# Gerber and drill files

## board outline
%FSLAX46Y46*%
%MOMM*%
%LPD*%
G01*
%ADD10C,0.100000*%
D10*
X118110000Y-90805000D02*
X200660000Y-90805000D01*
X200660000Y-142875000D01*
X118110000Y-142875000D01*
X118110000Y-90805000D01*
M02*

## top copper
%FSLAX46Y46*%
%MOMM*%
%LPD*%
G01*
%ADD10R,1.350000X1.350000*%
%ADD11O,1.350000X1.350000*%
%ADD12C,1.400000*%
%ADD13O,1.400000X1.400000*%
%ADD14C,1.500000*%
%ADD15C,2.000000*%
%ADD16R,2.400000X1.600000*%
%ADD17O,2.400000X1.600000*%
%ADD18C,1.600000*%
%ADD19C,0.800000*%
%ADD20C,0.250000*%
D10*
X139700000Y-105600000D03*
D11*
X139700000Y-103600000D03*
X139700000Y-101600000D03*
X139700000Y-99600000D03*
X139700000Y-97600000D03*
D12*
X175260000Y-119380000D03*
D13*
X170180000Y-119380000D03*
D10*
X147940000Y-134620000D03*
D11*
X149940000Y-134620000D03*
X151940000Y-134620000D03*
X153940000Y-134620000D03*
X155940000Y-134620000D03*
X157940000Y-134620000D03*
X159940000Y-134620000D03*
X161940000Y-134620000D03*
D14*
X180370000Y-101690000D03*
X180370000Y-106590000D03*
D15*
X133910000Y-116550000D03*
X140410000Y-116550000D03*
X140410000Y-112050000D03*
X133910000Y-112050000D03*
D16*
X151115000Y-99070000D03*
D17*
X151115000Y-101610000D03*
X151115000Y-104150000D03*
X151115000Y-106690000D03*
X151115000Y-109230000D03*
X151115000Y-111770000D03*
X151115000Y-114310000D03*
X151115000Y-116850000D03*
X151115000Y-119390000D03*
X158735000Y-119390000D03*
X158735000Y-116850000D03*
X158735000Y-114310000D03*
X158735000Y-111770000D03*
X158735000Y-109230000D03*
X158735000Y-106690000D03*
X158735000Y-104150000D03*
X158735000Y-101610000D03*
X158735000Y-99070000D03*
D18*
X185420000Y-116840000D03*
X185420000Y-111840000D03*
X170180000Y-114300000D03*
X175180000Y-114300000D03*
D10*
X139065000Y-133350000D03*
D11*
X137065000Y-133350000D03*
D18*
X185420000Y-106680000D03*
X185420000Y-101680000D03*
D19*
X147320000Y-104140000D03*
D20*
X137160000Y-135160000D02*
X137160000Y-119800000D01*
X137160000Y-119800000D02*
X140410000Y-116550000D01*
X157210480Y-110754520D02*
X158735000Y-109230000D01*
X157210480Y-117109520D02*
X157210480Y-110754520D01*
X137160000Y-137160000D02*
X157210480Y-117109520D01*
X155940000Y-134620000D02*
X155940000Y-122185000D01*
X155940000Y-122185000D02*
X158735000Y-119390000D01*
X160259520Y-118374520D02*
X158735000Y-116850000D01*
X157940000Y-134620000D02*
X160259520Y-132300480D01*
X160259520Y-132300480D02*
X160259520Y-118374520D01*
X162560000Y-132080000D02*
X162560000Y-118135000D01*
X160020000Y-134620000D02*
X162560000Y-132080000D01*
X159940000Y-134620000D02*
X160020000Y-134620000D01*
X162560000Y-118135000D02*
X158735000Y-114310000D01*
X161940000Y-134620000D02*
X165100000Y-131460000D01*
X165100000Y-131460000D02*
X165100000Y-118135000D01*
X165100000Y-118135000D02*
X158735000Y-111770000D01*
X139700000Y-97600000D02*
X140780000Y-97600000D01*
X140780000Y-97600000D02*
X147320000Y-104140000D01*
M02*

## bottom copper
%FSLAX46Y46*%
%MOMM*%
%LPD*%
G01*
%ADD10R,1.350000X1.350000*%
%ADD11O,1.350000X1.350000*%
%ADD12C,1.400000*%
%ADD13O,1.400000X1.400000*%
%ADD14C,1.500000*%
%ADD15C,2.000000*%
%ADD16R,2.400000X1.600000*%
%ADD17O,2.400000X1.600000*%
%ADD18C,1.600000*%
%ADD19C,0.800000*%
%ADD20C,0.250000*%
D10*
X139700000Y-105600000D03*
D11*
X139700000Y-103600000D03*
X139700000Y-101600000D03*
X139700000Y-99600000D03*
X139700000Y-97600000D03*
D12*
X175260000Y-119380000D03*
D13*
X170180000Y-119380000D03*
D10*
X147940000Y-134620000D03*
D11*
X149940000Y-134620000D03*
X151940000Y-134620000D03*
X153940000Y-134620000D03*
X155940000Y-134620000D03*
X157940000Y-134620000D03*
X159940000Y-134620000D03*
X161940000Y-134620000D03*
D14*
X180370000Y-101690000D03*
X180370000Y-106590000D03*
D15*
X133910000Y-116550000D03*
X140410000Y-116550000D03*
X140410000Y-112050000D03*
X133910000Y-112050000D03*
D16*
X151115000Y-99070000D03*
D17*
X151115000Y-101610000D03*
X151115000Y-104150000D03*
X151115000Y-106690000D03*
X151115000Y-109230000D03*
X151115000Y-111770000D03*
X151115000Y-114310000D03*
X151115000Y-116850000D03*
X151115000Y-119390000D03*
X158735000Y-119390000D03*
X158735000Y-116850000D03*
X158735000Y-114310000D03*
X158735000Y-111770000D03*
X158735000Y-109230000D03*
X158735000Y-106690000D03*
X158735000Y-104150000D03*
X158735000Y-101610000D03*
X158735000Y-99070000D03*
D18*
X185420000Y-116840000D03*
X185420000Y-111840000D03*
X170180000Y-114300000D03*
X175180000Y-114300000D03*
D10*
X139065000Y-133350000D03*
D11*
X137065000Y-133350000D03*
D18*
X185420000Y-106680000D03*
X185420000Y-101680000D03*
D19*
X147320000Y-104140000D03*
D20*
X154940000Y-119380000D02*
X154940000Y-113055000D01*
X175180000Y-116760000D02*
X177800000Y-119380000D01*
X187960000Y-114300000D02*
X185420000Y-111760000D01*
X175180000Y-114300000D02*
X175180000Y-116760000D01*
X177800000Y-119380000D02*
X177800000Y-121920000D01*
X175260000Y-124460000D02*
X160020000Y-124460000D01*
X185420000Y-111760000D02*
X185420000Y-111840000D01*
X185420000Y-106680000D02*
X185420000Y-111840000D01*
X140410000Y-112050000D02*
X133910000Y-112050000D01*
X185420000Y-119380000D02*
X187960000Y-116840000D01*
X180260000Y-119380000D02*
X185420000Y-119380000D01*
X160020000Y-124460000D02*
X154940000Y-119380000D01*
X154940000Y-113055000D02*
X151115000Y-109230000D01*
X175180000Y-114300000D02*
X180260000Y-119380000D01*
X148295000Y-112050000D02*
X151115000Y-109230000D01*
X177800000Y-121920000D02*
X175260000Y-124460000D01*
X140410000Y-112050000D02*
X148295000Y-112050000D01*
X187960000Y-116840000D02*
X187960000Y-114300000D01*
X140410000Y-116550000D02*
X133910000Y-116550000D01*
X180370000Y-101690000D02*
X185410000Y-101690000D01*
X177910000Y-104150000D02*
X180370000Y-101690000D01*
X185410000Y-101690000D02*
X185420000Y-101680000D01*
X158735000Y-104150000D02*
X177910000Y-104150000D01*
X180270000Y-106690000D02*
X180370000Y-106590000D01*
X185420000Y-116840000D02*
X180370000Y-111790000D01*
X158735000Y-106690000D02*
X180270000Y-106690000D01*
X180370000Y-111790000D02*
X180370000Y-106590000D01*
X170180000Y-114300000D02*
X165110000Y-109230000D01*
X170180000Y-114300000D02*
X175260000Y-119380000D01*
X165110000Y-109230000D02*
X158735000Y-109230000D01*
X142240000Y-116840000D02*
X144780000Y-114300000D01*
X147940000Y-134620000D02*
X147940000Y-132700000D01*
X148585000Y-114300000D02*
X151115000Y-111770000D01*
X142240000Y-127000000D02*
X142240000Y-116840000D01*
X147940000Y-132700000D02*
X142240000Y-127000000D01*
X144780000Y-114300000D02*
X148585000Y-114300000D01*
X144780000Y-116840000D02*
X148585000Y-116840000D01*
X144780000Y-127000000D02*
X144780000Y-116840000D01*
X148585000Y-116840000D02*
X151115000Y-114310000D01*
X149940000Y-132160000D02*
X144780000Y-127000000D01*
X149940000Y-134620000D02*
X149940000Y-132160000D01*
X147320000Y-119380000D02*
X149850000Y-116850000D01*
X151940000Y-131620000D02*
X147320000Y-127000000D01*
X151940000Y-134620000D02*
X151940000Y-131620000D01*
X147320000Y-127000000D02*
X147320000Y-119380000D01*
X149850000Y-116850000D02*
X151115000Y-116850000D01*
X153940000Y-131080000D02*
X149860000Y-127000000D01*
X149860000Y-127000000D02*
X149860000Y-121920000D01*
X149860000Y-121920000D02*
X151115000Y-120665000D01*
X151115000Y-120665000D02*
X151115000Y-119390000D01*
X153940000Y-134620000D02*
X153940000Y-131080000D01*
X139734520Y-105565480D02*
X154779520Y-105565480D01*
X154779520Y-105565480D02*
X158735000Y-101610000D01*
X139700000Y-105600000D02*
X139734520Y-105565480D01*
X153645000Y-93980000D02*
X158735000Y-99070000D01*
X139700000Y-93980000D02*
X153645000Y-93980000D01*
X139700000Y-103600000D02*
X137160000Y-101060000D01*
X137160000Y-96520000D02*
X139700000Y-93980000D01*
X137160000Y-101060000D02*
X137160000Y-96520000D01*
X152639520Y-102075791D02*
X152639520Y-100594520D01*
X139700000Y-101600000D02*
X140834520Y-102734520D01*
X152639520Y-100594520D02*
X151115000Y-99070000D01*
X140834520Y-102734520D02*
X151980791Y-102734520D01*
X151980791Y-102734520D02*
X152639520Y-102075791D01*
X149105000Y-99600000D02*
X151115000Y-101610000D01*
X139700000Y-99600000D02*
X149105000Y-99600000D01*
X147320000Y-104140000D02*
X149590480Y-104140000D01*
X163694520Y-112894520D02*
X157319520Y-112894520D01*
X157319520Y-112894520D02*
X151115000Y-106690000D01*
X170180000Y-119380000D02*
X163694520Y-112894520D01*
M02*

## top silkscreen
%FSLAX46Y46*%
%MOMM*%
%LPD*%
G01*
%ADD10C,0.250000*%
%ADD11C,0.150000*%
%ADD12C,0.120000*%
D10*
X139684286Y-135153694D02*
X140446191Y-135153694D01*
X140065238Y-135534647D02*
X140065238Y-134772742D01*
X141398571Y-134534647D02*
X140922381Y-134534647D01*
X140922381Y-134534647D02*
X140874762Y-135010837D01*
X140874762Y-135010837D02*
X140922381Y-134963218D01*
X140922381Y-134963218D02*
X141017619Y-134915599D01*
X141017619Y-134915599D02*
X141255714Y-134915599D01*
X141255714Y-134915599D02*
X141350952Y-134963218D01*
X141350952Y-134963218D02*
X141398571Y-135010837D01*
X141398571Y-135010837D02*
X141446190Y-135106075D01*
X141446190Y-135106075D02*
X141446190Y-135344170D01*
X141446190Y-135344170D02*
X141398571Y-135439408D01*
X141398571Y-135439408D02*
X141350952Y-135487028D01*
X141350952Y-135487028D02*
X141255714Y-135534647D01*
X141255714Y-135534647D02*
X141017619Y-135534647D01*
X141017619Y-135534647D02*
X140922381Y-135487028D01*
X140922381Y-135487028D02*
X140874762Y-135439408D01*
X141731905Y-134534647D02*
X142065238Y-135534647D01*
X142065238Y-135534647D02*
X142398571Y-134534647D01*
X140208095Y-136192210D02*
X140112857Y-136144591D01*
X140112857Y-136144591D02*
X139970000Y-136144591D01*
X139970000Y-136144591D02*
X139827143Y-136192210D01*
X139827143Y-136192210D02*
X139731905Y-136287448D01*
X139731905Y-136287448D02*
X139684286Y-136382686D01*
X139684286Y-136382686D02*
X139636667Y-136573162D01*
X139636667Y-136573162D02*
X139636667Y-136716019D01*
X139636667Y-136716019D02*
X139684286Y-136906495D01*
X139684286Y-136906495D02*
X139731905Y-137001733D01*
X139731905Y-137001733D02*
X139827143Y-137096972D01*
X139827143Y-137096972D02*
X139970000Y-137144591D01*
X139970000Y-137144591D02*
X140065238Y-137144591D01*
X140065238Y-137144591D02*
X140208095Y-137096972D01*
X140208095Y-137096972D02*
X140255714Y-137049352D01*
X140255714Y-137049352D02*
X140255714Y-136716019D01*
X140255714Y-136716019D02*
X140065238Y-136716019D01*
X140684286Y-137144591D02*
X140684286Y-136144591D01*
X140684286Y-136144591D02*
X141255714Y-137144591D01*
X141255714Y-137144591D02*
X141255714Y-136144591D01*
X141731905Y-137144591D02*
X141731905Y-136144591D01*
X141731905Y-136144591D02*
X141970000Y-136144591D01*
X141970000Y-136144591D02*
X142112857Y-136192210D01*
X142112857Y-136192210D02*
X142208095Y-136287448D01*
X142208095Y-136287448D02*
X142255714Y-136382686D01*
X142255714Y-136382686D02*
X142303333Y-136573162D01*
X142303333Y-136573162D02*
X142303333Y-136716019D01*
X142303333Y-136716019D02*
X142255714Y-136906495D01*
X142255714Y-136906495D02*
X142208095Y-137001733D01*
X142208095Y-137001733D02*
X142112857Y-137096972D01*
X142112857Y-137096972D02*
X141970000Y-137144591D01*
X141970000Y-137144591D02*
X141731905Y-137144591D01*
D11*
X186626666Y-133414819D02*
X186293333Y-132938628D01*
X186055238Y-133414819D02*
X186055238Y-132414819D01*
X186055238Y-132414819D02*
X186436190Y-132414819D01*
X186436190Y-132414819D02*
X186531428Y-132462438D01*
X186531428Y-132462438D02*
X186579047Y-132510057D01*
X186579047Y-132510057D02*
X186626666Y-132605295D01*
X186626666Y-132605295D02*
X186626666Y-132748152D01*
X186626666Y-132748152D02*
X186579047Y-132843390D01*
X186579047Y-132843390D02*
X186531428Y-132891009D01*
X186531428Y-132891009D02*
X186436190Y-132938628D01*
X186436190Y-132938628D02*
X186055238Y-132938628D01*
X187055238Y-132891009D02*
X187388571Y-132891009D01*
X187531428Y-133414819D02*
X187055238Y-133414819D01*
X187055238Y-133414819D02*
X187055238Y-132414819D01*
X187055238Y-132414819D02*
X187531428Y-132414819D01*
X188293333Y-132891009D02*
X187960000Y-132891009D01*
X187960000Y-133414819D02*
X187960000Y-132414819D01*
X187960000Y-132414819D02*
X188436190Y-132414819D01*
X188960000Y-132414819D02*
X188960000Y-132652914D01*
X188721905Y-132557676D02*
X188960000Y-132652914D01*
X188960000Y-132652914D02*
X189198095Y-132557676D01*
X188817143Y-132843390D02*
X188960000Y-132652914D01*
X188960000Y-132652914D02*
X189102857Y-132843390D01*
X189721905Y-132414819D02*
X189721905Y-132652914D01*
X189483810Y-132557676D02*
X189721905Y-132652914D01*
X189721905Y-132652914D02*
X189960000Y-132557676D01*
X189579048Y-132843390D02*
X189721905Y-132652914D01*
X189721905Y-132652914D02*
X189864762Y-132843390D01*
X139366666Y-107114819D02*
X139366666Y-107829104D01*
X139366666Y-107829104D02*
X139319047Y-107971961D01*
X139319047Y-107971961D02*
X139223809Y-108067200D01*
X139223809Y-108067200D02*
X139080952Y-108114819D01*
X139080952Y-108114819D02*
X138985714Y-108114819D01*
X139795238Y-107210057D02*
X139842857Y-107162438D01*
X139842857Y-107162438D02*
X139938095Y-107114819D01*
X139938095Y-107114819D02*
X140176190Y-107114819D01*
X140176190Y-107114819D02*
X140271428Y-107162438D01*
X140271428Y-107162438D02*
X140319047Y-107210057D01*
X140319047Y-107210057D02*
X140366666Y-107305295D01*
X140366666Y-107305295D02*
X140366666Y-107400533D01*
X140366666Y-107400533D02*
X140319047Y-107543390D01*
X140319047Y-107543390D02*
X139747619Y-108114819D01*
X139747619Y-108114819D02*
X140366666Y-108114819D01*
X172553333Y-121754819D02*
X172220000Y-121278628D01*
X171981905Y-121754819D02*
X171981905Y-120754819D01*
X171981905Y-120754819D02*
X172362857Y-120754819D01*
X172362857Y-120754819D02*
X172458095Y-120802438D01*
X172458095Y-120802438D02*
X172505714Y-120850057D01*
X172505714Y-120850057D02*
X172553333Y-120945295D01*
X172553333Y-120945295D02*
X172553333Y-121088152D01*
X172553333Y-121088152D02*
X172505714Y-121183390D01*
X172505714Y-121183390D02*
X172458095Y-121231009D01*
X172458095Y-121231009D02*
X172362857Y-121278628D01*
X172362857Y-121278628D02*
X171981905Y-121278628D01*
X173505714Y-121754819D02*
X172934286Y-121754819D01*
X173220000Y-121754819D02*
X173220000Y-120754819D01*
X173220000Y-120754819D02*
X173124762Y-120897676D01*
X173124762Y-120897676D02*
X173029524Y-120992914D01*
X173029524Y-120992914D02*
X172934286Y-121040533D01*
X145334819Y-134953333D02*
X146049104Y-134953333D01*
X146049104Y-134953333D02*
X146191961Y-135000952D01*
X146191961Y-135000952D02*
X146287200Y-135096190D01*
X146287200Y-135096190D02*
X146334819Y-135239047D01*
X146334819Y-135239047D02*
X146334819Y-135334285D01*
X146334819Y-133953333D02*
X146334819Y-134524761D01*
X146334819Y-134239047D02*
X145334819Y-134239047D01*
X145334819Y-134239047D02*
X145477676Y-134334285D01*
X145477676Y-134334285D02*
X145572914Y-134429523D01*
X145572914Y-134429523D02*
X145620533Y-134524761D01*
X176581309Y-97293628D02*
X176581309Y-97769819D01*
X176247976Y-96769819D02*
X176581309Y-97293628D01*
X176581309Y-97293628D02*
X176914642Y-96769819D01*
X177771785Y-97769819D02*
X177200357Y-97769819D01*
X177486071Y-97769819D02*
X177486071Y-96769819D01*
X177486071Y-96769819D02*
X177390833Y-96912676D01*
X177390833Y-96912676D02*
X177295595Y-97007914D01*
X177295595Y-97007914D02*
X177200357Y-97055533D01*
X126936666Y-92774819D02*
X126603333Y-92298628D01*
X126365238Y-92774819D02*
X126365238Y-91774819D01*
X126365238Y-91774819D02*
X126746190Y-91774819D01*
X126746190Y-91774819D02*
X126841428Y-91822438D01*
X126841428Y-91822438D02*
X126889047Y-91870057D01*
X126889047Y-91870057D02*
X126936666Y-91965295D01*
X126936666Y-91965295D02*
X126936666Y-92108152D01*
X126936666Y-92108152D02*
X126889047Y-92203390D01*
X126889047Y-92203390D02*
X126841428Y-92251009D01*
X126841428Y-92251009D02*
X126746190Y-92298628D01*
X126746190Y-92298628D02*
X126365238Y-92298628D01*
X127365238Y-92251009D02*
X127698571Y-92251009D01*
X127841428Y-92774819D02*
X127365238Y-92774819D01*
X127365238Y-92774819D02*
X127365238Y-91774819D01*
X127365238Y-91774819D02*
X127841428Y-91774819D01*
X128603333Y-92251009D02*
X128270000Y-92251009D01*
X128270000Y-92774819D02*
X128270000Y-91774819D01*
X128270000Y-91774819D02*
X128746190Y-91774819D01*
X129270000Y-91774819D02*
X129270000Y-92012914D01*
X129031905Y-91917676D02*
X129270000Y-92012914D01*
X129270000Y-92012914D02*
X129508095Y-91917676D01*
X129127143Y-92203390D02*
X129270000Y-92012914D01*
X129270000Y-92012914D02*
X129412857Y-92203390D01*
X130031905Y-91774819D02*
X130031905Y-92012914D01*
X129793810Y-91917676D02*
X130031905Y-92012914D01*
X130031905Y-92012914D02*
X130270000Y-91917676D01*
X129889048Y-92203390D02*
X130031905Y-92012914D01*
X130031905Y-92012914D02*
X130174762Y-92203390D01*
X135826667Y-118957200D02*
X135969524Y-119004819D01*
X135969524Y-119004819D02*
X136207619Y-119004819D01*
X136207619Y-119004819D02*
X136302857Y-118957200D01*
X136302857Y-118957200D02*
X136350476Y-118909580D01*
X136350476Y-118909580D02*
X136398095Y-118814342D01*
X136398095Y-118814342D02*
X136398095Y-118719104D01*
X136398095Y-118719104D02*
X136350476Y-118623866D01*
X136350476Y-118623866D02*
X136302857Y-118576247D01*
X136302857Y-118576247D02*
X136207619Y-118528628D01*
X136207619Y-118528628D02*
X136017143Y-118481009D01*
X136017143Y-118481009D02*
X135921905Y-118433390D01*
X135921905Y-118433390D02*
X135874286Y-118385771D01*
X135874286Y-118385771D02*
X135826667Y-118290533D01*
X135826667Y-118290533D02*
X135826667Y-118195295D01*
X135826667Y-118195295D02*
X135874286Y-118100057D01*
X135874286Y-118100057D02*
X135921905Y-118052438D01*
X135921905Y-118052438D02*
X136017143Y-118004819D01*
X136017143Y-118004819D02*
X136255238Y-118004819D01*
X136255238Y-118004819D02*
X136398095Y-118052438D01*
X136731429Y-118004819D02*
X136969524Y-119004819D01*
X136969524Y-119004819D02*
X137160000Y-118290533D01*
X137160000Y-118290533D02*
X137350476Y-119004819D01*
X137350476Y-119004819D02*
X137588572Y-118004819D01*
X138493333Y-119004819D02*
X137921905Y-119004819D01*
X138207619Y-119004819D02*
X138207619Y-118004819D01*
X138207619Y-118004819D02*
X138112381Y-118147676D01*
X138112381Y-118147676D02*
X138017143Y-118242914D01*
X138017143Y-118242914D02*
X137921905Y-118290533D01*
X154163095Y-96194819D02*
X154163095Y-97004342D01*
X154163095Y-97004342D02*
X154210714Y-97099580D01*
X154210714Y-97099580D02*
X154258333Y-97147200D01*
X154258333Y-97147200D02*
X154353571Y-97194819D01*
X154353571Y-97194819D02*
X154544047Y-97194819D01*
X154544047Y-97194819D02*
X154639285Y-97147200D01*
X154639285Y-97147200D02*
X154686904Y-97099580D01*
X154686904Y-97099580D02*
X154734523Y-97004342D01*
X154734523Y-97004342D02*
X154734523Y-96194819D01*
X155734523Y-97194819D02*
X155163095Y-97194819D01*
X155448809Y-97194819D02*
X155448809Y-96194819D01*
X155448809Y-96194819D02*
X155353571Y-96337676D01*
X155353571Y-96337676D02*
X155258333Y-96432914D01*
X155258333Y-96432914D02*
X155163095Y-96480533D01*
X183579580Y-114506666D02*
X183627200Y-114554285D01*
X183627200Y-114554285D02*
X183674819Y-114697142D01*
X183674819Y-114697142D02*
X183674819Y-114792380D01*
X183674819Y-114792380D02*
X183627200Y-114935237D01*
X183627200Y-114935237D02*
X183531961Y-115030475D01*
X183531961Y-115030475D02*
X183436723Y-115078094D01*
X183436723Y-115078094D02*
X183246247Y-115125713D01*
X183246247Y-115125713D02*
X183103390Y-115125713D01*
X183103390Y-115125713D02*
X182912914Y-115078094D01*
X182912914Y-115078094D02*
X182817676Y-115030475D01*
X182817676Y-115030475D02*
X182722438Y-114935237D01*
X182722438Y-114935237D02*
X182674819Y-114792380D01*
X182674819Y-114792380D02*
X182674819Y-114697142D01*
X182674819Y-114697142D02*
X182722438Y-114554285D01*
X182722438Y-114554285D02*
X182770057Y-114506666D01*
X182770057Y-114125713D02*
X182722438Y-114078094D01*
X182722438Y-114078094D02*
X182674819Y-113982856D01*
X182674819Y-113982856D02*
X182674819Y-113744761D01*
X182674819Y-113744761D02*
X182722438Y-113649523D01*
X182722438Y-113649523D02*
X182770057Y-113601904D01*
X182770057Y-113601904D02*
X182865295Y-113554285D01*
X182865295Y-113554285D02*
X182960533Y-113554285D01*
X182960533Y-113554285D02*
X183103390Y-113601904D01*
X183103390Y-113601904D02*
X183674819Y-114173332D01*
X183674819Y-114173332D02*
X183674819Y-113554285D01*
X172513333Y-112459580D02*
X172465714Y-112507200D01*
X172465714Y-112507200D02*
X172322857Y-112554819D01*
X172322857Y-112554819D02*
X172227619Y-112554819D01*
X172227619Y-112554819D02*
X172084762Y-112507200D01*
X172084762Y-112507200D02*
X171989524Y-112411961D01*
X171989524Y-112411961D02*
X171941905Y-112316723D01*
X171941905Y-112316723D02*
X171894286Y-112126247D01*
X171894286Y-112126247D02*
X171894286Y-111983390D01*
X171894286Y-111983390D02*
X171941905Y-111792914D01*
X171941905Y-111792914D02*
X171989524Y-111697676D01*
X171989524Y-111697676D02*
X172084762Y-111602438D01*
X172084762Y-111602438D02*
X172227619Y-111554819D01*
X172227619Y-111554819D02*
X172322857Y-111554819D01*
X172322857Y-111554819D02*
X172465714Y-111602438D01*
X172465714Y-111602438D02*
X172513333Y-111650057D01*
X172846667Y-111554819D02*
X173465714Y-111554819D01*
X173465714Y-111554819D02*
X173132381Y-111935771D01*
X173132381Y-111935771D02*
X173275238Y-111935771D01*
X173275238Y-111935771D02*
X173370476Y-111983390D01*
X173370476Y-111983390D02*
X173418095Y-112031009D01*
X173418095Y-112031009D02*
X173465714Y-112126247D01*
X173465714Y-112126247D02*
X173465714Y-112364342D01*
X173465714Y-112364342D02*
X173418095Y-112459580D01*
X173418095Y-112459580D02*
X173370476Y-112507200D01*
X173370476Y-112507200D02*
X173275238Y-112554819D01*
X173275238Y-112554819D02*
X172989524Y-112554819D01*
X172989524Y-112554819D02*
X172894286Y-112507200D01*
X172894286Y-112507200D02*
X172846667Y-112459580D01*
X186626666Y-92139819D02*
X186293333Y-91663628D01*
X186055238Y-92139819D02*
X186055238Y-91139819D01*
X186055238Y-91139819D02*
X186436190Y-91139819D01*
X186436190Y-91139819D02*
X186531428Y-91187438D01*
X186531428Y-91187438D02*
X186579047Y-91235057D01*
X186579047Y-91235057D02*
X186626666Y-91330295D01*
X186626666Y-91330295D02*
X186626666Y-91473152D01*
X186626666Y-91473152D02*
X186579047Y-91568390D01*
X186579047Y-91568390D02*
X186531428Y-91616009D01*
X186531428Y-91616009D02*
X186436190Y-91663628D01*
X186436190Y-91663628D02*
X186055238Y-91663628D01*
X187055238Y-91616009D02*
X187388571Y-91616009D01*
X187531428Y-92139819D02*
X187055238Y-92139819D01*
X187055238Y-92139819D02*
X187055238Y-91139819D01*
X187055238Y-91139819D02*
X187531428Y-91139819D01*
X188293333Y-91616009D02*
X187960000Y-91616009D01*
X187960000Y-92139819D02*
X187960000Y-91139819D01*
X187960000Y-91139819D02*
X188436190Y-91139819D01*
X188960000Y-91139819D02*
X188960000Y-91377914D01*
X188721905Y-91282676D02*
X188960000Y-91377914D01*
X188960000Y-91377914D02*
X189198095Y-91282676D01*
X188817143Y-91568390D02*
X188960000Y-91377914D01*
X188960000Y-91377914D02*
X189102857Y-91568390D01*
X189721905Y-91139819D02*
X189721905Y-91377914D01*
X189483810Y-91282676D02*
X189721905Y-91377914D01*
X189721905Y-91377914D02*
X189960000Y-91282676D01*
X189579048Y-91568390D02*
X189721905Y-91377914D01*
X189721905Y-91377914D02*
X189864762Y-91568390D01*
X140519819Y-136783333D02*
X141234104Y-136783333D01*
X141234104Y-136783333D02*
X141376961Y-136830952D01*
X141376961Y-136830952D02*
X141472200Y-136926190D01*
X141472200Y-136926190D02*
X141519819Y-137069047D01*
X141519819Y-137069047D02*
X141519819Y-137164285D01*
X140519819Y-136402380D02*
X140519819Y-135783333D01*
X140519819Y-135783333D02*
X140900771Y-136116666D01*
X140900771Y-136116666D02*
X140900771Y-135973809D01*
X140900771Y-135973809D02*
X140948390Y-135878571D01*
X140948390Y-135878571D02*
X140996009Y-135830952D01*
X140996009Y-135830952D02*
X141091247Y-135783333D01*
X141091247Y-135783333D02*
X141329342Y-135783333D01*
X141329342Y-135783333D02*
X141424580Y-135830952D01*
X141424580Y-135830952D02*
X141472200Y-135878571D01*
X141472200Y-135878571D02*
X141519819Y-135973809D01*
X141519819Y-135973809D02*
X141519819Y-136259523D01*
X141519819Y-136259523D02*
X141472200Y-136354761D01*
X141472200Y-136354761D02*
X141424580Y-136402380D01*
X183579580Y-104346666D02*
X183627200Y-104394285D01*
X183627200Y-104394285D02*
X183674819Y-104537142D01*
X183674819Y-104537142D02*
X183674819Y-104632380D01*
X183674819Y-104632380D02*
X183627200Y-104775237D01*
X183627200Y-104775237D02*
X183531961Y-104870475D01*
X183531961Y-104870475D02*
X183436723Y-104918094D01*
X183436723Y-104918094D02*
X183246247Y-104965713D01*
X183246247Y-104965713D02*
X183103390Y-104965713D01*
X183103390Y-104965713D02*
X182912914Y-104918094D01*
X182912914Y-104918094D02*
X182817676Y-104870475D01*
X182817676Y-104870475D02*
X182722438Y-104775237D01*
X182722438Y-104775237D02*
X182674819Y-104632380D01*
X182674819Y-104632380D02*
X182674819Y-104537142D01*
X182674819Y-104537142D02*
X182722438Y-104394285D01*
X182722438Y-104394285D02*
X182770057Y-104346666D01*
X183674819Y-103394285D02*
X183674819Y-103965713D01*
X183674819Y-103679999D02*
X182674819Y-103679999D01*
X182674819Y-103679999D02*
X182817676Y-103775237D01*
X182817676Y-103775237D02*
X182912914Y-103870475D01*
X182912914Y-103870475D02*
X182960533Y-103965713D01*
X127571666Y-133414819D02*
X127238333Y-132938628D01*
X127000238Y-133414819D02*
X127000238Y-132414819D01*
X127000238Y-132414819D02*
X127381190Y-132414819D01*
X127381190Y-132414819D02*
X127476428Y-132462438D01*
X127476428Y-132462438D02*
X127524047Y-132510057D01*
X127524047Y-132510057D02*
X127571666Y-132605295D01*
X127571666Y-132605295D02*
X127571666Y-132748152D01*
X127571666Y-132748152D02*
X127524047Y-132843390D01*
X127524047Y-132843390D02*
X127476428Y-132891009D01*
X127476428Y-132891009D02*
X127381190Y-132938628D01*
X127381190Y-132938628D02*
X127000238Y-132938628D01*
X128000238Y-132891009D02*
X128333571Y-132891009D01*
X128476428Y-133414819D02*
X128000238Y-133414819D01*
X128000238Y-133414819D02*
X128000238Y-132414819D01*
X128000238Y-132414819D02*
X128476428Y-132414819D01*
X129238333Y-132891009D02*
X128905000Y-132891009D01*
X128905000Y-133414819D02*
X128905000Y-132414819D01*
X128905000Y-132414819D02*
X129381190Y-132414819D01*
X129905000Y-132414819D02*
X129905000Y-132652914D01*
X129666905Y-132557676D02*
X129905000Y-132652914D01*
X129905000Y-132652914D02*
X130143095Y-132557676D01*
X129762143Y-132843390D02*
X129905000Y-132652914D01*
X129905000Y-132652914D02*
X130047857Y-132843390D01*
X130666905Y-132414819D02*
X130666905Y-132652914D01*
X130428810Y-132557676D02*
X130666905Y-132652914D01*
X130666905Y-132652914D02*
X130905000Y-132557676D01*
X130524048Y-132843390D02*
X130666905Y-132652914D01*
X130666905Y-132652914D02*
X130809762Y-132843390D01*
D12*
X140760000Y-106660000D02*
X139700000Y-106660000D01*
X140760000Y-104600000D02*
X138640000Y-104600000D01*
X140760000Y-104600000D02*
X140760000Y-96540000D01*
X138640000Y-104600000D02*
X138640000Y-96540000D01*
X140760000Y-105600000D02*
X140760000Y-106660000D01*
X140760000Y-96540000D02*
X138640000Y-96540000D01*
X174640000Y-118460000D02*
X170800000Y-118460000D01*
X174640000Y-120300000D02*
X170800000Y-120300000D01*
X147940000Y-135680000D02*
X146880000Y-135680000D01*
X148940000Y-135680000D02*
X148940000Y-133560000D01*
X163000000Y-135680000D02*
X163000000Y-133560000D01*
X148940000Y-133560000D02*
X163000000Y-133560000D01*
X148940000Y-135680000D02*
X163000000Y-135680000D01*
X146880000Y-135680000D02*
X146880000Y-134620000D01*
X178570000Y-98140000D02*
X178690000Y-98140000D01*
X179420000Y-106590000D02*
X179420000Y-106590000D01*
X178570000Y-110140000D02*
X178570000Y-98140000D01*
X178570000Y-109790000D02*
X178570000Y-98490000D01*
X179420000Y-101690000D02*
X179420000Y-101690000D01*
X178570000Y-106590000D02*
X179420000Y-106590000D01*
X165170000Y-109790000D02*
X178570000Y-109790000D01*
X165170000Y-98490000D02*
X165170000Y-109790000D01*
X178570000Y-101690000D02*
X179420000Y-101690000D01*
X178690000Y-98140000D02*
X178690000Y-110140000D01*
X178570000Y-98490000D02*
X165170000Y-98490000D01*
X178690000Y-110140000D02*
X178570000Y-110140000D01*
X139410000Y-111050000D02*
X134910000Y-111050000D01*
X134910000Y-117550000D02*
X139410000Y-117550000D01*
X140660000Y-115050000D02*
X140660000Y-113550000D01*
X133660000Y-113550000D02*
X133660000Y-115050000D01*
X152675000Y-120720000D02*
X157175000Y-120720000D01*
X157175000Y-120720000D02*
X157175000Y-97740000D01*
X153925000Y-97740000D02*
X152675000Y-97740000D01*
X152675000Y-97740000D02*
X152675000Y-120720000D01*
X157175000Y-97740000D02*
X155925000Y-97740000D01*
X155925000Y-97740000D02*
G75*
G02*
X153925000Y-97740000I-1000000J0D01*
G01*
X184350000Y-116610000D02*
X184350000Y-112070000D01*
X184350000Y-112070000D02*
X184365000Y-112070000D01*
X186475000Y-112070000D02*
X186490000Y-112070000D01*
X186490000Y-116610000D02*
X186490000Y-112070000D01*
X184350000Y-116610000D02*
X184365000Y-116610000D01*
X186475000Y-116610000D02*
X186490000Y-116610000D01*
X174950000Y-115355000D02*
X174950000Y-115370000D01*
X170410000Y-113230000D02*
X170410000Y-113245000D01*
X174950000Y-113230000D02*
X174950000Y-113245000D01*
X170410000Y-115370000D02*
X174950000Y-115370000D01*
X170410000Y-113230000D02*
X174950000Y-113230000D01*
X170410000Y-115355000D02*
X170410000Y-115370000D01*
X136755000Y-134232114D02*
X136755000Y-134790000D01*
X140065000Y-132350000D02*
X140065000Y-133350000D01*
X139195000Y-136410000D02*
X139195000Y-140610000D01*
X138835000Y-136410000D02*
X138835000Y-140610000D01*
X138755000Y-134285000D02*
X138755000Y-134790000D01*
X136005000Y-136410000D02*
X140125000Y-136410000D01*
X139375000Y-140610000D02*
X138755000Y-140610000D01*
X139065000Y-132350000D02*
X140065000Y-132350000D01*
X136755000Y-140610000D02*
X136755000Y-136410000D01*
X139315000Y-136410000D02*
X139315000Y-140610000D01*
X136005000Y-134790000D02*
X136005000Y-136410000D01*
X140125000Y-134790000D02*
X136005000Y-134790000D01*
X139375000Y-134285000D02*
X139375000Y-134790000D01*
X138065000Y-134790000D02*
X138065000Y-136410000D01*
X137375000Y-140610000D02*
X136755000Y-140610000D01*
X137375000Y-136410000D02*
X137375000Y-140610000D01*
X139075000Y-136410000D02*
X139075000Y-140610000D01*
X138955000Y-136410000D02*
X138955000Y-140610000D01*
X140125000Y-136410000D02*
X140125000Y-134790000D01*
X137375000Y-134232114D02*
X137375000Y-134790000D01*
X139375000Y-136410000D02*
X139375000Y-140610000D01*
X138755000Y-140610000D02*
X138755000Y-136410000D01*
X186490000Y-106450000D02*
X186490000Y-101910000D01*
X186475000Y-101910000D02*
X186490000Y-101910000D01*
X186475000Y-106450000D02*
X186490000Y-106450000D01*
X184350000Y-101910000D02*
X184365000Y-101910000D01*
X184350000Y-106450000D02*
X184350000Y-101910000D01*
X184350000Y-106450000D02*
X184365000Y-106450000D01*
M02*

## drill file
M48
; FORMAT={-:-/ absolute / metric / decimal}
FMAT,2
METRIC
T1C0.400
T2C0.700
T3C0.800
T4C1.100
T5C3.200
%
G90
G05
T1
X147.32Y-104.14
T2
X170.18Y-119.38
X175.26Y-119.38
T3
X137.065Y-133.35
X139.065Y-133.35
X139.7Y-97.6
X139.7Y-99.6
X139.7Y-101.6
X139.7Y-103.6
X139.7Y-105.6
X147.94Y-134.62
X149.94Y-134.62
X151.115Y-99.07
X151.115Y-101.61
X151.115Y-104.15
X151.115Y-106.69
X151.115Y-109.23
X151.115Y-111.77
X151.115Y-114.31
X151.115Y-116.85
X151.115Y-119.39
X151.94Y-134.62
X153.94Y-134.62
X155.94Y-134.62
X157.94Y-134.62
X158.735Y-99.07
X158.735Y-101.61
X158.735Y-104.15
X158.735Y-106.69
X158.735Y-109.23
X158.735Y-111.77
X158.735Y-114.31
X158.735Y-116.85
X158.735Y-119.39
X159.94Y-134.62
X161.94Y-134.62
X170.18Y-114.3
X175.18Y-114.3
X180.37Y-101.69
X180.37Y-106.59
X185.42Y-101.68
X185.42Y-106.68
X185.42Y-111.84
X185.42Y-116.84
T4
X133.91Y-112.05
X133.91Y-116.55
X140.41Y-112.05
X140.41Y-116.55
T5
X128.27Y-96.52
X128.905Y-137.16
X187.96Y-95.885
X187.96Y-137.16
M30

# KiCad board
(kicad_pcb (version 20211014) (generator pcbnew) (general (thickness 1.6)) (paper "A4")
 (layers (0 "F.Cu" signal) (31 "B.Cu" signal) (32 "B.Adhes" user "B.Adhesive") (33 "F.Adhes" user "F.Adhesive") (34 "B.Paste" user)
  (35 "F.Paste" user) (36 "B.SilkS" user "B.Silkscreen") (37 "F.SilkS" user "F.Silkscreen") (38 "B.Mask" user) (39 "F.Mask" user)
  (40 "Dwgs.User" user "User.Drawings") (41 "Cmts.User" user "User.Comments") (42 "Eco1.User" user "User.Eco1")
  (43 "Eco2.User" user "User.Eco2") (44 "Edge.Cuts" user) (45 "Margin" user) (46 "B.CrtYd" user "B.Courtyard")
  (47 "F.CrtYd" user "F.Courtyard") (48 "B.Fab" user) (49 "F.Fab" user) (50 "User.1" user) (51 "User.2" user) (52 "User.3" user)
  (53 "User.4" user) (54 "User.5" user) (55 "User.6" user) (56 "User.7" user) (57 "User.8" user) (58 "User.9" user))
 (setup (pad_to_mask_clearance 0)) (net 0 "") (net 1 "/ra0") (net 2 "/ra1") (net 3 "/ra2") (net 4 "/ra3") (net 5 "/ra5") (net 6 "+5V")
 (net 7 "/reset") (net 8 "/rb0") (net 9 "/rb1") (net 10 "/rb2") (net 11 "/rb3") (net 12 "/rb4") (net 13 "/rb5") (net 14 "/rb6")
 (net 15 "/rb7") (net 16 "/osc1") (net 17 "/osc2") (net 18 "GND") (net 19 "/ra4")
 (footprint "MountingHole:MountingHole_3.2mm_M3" (layer "F.Cu") (at 187.96 137.16)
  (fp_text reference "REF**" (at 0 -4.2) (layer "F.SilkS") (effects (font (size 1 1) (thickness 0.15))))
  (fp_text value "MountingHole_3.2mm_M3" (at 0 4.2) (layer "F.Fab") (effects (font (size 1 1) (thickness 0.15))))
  (pad "" np_thru_hole circle (at 0 0) (size 3.2 3.2) (drill 3.2) (layers *.Cu *.Mask)))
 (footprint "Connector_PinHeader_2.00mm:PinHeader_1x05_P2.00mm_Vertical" (layer "F.Cu") (at 139.7 105.6 180)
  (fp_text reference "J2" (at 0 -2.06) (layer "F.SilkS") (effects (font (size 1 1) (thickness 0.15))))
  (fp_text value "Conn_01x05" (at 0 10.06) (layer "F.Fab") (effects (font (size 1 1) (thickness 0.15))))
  (fp_line (start -1.06 -1.06) (end 0 -1.06) (layer "F.SilkS") (width 0.12))
  (fp_line (start -1.06 1) (end 1.06 1) (layer "F.SilkS") (width 0.12))
  (fp_line (start -1.06 1) (end -1.06 9.06) (layer "F.SilkS") (width 0.12))
  (fp_line (start 1.06 1) (end 1.06 9.06) (layer "F.SilkS") (width 0.12))
  (fp_line (start -1.06 0) (end -1.06 -1.06) (layer "F.SilkS") (width 0.12))
  (fp_line (start -1.06 9.06) (end 1.06 9.06) (layer "F.SilkS") (width 0.12))
  (pad "1" thru_hole rect (at 0 0 180) (size 1.35 1.35) (drill 0.8) (layers *.Cu *.Mask) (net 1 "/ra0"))
  (pad "2" thru_hole oval (at 0 2 180) (size 1.35 1.35) (drill 0.8) (layers *.Cu *.Mask) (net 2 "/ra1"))
  (pad "3" thru_hole oval (at 0 4 180) (size 1.35 1.35) (drill 0.8) (layers *.Cu *.Mask) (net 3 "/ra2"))
  (pad "4" thru_hole oval (at 0 6 180) (size 1.35 1.35) (drill 0.8) (layers *.Cu *.Mask) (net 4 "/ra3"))
  (pad "5" thru_hole oval (at 0 8 180) (size 1.35 1.35) (drill 0.8) (layers *.Cu *.Mask) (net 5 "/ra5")))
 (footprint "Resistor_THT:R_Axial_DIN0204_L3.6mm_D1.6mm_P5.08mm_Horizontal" (layer "F.Cu") (at 175.26 119.38 180)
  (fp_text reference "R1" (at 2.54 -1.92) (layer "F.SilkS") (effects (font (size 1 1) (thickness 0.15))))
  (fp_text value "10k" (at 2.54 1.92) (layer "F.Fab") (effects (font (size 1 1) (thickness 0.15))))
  (fp_line (start 0.62 0.92) (end 4.46 0.92) (layer "F.SilkS") (width 0.12))
  (fp_line (start 0.62 -0.92) (end 4.46 -0.92) (layer "F.SilkS") (width 0.12))
  (pad "1" thru_hole circle (at 0 0 180) (size 1.4 1.4) (drill 0.7) (layers *.Cu *.Mask) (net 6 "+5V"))
  (pad "2" thru_hole oval (at 5.08 0 180) (size 1.4 1.4) (drill 0.7) (layers *.Cu *.Mask) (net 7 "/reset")))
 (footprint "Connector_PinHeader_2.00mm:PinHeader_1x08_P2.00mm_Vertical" (layer "F.Cu") (at 147.94 134.62 90)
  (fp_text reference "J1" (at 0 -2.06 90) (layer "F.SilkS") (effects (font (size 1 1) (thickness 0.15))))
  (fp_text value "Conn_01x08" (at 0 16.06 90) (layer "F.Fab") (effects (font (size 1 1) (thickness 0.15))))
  (fp_line (start -1.06 0) (end -1.06 -1.06) (layer "F.SilkS") (width 0.12))
  (fp_line (start -1.06 1) (end 1.06 1) (layer "F.SilkS") (width 0.12))
  (fp_line (start -1.06 15.06) (end 1.06 15.06) (layer "F.SilkS") (width 0.12))
  (fp_line (start 1.06 1) (end 1.06 15.06) (layer "F.SilkS") (width 0.12))
  (fp_line (start -1.06 1) (end -1.06 15.06) (layer "F.SilkS") (width 0.12))
  (fp_line (start -1.06 -1.06) (end 0 -1.06) (layer "F.SilkS") (width 0.12))
  (pad "1" thru_hole rect (at 0 0 90) (size 1.35 1.35) (drill 0.8) (layers *.Cu *.Mask) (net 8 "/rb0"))
  (pad "2" thru_hole oval (at 0 2 90) (size 1.35 1.35) (drill 0.8) (layers *.Cu *.Mask) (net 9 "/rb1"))
  (pad "3" thru_hole oval (at 0 4 90) (size 1.35 1.35) (drill 0.8) (layers *.Cu *.Mask) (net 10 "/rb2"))
  (pad "4" thru_hole oval (at 0 6 90) (size 1.35 1.35) (drill 0.8) (layers *.Cu *.Mask) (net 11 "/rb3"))
  (pad "5" thru_hole oval (at 0 8 90) (size 1.35 1.35) (drill 0.8) (layers *.Cu *.Mask) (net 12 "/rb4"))
  (pad "6" thru_hole oval (at 0 10 90) (size 1.35 1.35) (drill 0.8) (layers *.Cu *.Mask) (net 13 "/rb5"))
  (pad "7" thru_hole oval (at 0 12 90) (size 1.35 1.35) (drill 0.8) (layers *.Cu *.Mask) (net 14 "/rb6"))
  (pad "8" thru_hole oval (at 0 14 90) (size 1.35 1.35) (drill 0.8) (layers *.Cu *.Mask) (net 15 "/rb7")))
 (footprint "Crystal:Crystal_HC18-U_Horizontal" (layer "F.Cu") (at 180.37 101.69 -90)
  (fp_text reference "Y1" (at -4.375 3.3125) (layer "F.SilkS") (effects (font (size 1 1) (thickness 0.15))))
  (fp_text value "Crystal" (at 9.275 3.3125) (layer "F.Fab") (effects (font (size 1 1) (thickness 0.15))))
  (fp_line (start -3.55 1.8) (end -3.55 1.68) (layer "F.SilkS") (width 0.12))
  (fp_line (start 4.9 0.95) (end 4.9 0.95) (layer "F.SilkS") (width 0.12))
  (fp_line (start 8.45 1.8) (end -3.55 1.8) (layer "F.SilkS") (width 0.12))
  (fp_line (start 8.1 1.8) (end -3.2 1.8) (layer "F.SilkS") (width 0.12))
  (fp_line (start 0 0.95) (end 0 0.95) (layer "F.SilkS") (width 0.12))
  (fp_line (start 4.9 1.8) (end 4.9 0.95) (layer "F.SilkS") (width 0.12))
  (fp_line (start 8.1 15.2) (end 8.1 1.8) (layer "F.SilkS") (width 0.12))
  (fp_line (start -3.2 15.2) (end 8.1 15.2) (layer "F.SilkS") (width 0.12))
  (fp_line (start 0 1.8) (end 0 0.95) (layer "F.SilkS") (width 0.12))
  (fp_line (start -3.55 1.68) (end 8.45 1.68) (layer "F.SilkS") (width 0.12))
  (fp_line (start -3.2 1.8) (end -3.2 15.2) (layer "F.SilkS") (width 0.12))
  (fp_line (start 8.45 1.68) (end 8.45 1.8) (layer "F.SilkS") (width 0.12))
  (pad "1" thru_hole circle (at 0 0 270) (size 1.5 1.5) (drill 0.8) (layers *.Cu *.Mask) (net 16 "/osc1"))
  (pad "2" thru_hole circle (at 4.9 0 270) (size 1.5 1.5) (drill 0.8) (layers *.Cu *.Mask) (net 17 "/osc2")))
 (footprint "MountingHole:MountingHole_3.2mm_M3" (layer "F.Cu") (at 128.27 96.52)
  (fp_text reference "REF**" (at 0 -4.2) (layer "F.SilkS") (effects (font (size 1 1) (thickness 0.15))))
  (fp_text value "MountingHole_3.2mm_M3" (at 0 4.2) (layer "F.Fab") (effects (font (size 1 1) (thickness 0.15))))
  (pad "" np_thru_hole circle (at 0 0) (size 3.2 3.2) (drill 3.2) (layers *.Cu *.Mask)))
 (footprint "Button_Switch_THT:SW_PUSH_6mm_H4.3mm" (layer "F.Cu") (at 140.41 116.55 180)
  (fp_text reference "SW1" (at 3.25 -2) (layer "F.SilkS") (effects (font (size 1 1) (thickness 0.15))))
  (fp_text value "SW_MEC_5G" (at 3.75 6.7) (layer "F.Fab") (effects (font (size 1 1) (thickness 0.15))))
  (fp_line (start 1 5.5) (end 5.5 5.5) (layer "F.SilkS") (width 0.12))
  (fp_line (start 5.5 -1) (end 1 -1) (layer "F.SilkS") (width 0.12))
  (fp_line (start -0.25 1.5) (end -0.25 3) (layer "F.SilkS") (width 0.12))
  (fp_line (start 6.75 3) (end 6.75 1.5) (layer "F.SilkS") (width 0.12))
  (pad "1" thru_hole circle (at 6.5 0 270) (size 2 2) (drill 1.1) (layers *.Cu *.Mask) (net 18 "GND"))
  (pad "1" thru_hole circle (at 0 0 270) (size 2 2) (drill 1.1) (layers *.Cu *.Mask) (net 18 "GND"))
  (pad "2" thru_hole circle (at 0 4.5 270) (size 2 2) (drill 1.1) (layers *.Cu *.Mask) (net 18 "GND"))
  (pad "2" thru_hole circle (at 6.5 4.5 270) (size 2 2) (drill 1.1) (layers *.Cu *.Mask) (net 18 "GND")))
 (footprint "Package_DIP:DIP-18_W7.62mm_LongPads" (layer "F.Cu") (at 151.115 99.07)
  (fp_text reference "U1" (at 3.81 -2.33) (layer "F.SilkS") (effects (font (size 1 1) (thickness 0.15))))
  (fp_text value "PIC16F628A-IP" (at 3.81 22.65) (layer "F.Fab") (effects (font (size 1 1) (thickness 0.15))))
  (fp_line (start 1.56 21.65) (end 6.06 21.65) (layer "F.SilkS") (width 0.12))
  (fp_line (start 6.06 21.65) (end 6.06 -1.33) (layer "F.SilkS") (width 0.12))
  (fp_line (start 2.81 -1.33) (end 1.56 -1.33) (layer "F.SilkS") (width 0.12))
  (fp_line (start 1.56 -1.33) (end 1.56 21.65) (layer "F.SilkS") (width 0.12))
  (fp_line (start 6.06 -1.33) (end 4.81 -1.33) (layer "F.SilkS") (width 0.12))
  (fp_arc (start 4.81 -1.33) (mid 3.81 -0.33) (end 2.81 -1.33) (layer "F.SilkS") (width 0.12))
  (pad "1" thru_hole rect (at 0 0) (size 2.4 1.6) (drill 0.8) (layers *.Cu *.Mask) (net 3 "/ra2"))
  (pad "2" thru_hole oval (at 0 2.54) (size 2.4 1.6) (drill 0.8) (layers *.Cu *.Mask) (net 4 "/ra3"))
  (pad "3" thru_hole oval (at 0 5.08) (size 2.4 1.6) (drill 0.8) (layers *.Cu *.Mask) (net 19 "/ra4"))
  (pad "4" thru_hole oval (at 0 7.62) (size 2.4 1.6) (drill 0.8) (layers *.Cu *.Mask) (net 7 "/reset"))
  (pad "5" thru_hole oval (at 0 10.16) (size 2.4 1.6) (drill 0.8) (layers *.Cu *.Mask) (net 18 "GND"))
  (pad "6" thru_hole oval (at 0 12.7) (size 2.4 1.6) (drill 0.8) (layers *.Cu *.Mask) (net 8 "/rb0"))
  (pad "7" thru_hole oval (at 0 15.24) (size 2.4 1.6) (drill 0.8) (layers *.Cu *.Mask) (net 9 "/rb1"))
  (pad "8" thru_hole oval (at 0 17.78) (size 2.4 1.6) (drill 0.8) (layers *.Cu *.Mask) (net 10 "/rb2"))
  (pad "9" thru_hole oval (at 0 20.32) (size 2.4 1.6) (drill 0.8) (layers *.Cu *.Mask) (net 11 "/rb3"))
  (pad "10" thru_hole oval (at 7.62 20.32) (size 2.4 1.6) (drill 0.8) (layers *.Cu *.Mask) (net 12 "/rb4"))
  (pad "11" thru_hole oval (at 7.62 17.78) (size 2.4 1.6) (drill 0.8) (layers *.Cu *.Mask) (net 13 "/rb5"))
  (pad "12" thru_hole oval (at 7.62 15.24) (size 2.4 1.6) (drill 0.8) (layers *.Cu *.Mask) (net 14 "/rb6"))
  (pad "13" thru_hole oval (at 7.62 12.7) (size 2.4 1.6) (drill 0.8) (layers *.Cu *.Mask) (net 15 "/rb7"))
  (pad "14" thru_hole oval (at 7.62 10.16) (size 2.4 1.6) (drill 0.8) (layers *.Cu *.Mask) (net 6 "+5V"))
  (pad "15" thru_hole oval (at 7.62 7.62) (size 2.4 1.6) (drill 0.8) (layers *.Cu *.Mask) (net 17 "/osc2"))
  (pad "16" thru_hole oval (at 7.62 5.08) (size 2.4 1.6) (drill 0.8) (layers *.Cu *.Mask) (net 16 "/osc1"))
  (pad "17" thru_hole oval (at 7.62 2.54) (size 2.4 1.6) (drill 0.8) (layers *.Cu *.Mask) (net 1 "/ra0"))
  (pad "18" thru_hole oval (at 7.62 0) (size 2.4 1.6) (drill 0.8) (layers *.Cu *.Mask) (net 2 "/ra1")))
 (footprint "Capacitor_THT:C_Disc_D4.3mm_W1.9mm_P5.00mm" (layer "F.Cu") (at 185.42 116.84 90)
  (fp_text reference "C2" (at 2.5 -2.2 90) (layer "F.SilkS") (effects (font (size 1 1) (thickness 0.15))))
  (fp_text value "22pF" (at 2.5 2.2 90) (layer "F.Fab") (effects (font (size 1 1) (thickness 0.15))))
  (fp_line (start 0.23 -1.07) (end 4.77 -1.07) (layer "F.SilkS") (width 0.12))
  (fp_line (start 4.77 -1.07) (end 4.77 -1.055) (layer "F.SilkS") (width 0.12))
  (fp_line (start 4.77 1.055) (end 4.77 1.07) (layer "F.SilkS") (width 0.12))
  (fp_line (start 0.23 1.07) (end 4.77 1.07) (layer "F.SilkS") (width 0.12))
  (fp_line (start 0.23 -1.07) (end 0.23 -1.055) (layer "F.SilkS") (width 0.12))
  (fp_line (start 0.23 1.055) (end 0.23 1.07) (layer "F.SilkS") (width 0.12))
  (pad "1" thru_hole circle (at 0 0 90) (size 1.6 1.6) (drill 0.8) (layers *.Cu *.Mask) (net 17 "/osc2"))
  (pad "2" thru_hole circle (at 5 0 90) (size 1.6 1.6) (drill 0.8) (layers *.Cu *.Mask) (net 18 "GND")))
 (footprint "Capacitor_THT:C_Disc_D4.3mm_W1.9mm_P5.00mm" (layer "F.Cu") (at 170.18 114.3)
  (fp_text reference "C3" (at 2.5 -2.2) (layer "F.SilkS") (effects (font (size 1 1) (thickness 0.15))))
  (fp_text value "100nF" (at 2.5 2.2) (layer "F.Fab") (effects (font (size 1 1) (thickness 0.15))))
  (fp_line (start 4.77 1.055) (end 4.77 1.07) (layer "F.SilkS") (width 0.12))
  (fp_line (start 0.23 -1.07) (end 0.23 -1.055) (layer "F.SilkS") (width 0.12))
  (fp_line (start 4.77 -1.07) (end 4.77 -1.055) (layer "F.SilkS") (width 0.12))
  (fp_line (start 0.23 1.07) (end 4.77 1.07) (layer "F.SilkS") (width 0.12))
  (fp_line (start 0.23 -1.07) (end 4.77 -1.07) (layer "F.SilkS") (width 0.12))
  (fp_line (start 0.23 1.055) (end 0.23 1.07) (layer "F.SilkS") (width 0.12))
  (pad "1" thru_hole circle (at 0 0) (size 1.6 1.6) (drill 0.8) (layers *.Cu *.Mask) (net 6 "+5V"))
  (pad "2" thru_hole circle (at 5 0) (size 1.6 1.6) (drill 0.8) (layers *.Cu *.Mask) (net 18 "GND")))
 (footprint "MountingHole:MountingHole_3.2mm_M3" (layer "F.Cu") (at 187.96 95.885)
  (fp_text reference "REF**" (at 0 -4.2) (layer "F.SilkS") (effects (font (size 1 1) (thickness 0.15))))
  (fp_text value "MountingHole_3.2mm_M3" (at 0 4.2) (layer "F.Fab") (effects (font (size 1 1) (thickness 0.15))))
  (pad "" np_thru_hole circle (at 0 0) (size 3.2 3.2) (drill 3.2) (layers *.Cu *.Mask)))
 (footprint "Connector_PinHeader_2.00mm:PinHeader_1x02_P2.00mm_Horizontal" (layer "F.Cu") (at 139.065 133.35 -90)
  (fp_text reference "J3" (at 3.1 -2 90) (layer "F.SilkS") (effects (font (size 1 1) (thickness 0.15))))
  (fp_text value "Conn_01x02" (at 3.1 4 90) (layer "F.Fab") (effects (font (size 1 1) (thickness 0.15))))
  (fp_line (start 0.882114 2.31) (end 1.44 2.31) (layer "F.SilkS") (width 0.12))
  (fp_line (start -1 -1) (end 0 -1) (layer "F.SilkS") (width 0.12))
  (fp_line (start 3.06 -0.13) (end 7.26 -0.13) (layer "F.SilkS") (width 0.12))
  (fp_line (start 3.06 0.23) (end 7.26 0.23) (layer "F.SilkS") (width 0.12))
  (fp_line (start 0.935 0.31) (end 1.44 0.31) (layer "F.SilkS") (width 0.12))
  (fp_line (start 3.06 3.06) (end 3.06 -1.06) (layer "F.SilkS") (width 0.12))
  (fp_line (start 7.26 -0.31) (end 7.26 0.31) (layer "F.SilkS") (width 0.12))
  (fp_line (start -1 0) (end -1 -1) (layer "F.SilkS") (width 0.12))
  (fp_line (start 7.26 2.31) (end 3.06 2.31) (layer "F.SilkS") (width 0.12))
  (fp_line (start 3.06 -0.25) (end 7.26 -0.25) (layer "F.SilkS") (width 0.12))
  (fp_line (start 1.44 3.06) (end 3.06 3.06) (layer "F.SilkS") (width 0.12))
  (fp_line (start 1.44 -1.06) (end 1.44 3.06) (layer "F.SilkS") (width 0.12))
  (fp_line (start 0.935 -0.31) (end 1.44 -0.31) (layer "F.SilkS") (width 0.12))
  (fp_line (start 1.44 1) (end 3.06 1) (layer "F.SilkS") (width 0.12))
  (fp_line (start 7.26 1.69) (end 7.26 2.31) (layer "F.SilkS") (width 0.12))
  (fp_line (start 3.06 1.69) (end 7.26 1.69) (layer "F.SilkS") (width 0.12))
  (fp_line (start 3.06 -0.01) (end 7.26 -0.01) (layer "F.SilkS") (width 0.12))
  (fp_line (start 3.06 0.11) (end 7.26 0.11) (layer "F.SilkS") (width 0.12))
  (fp_line (start 3.06 -1.06) (end 1.44 -1.06) (layer "F.SilkS") (width 0.12))
  (fp_line (start 0.882114 1.69) (end 1.44 1.69) (layer "F.SilkS") (width 0.12))
  (fp_line (start 3.06 -0.31) (end 7.26 -0.31) (layer "F.SilkS") (width 0.12))
  (fp_line (start 7.26 0.31) (end 3.06 0.31) (layer "F.SilkS") (width 0.12))
  (pad "1" thru_hole rect (at 0 0 270) (size 1.35 1.35) (drill 0.8) (layers *.Cu *.Mask) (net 6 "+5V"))
  (pad "2" thru_hole oval (at 0 2 270) (size 1.35 1.35) (drill 0.8) (layers *.Cu *.Mask) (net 18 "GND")))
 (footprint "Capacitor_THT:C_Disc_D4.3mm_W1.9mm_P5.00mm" (layer "F.Cu") (at 185.42 106.68 90)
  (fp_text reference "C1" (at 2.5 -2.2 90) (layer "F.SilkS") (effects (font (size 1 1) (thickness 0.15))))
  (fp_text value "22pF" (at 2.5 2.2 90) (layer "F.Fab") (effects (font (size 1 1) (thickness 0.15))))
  (fp_line (start 0.23 1.07) (end 4.77 1.07) (layer "F.SilkS") (width 0.12))
  (fp_line (start 4.77 1.055) (end 4.77 1.07) (layer "F.SilkS") (width 0.12))
  (fp_line (start 0.23 1.055) (end 0.23 1.07) (layer "F.SilkS") (width 0.12))
  (fp_line (start 4.77 -1.07) (end 4.77 -1.055) (layer "F.SilkS") (width 0.12))
  (fp_line (start 0.23 -1.07) (end 4.77 -1.07) (layer "F.SilkS") (width 0.12))
  (fp_line (start 0.23 -1.07) (end 0.23 -1.055) (layer "F.SilkS") (width 0.12))
  (pad "1" thru_hole circle (at 0 0 90) (size 1.6 1.6) (drill 0.8) (layers *.Cu *.Mask) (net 18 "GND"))
  (pad "2" thru_hole circle (at 5 0 90) (size 1.6 1.6) (drill 0.8) (layers *.Cu *.Mask) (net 16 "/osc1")))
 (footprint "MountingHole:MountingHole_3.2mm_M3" (layer "F.Cu") (at 128.905 137.16)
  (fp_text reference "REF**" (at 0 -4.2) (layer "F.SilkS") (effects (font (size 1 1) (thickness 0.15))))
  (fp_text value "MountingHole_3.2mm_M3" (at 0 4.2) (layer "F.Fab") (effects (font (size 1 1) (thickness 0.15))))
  (pad "" np_thru_hole circle (at 0 0) (size 3.2 3.2) (drill 3.2) (layers *.Cu *.Mask)))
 (gr_rect (start 118.11 90.805) (end 200.66 142.875) (layer "Edge.Cuts") (width 0.1) (fill none))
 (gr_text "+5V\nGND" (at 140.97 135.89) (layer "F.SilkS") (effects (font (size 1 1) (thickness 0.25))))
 (segment (start 137.16 135.16) (end 137.16 119.8) (width 0.25) (layer "F.Cu") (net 18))
 (segment (start 137.16 119.8) (end 140.41 116.55) (width 0.25) (layer "F.Cu") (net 18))
 (segment (start 154.94 119.38) (end 154.94 113.055) (width 0.25) (layer "B.Cu") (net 18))
 (segment (start 175.18 116.76) (end 177.8 119.38) (width 0.25) (layer "B.Cu") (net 18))
 (segment (start 187.96 114.3) (end 185.42 111.76) (width 0.25) (layer "B.Cu") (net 18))
 (segment (start 175.18 114.3) (end 175.18 116.76) (width 0.25) (layer "B.Cu") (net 18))
 (segment (start 177.8 119.38) (end 177.8 121.92) (width 0.25) (layer "B.Cu") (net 18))
 (segment (start 175.26 124.46) (end 160.02 124.46) (width 0.25) (layer "B.Cu") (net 18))
 (segment (start 185.42 111.76) (end 185.42 111.84) (width 0.25) (layer "B.Cu") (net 18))
 (segment (start 185.42 106.68) (end 185.42 111.84) (width 0.25) (layer "B.Cu") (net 18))
 (segment (start 140.41 112.05) (end 133.91 112.05) (width 0.25) (layer "B.Cu") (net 18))
 (segment (start 185.42 119.38) (end 187.96 116.84) (width 0.25) (layer "B.Cu") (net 18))
 (segment (start 180.26 119.38) (end 185.42 119.38) (width 0.25) (layer "B.Cu") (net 18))
 (segment (start 160.02 124.46) (end 154.94 119.38) (width 0.25) (layer "B.Cu") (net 18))
 (segment (start 154.94 113.055) (end 151.115 109.23) (width 0.25) (layer "B.Cu") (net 18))
 (segment (start 175.18 114.3) (end 180.26 119.38) (width 0.25) (layer "B.Cu") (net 18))
 (segment (start 148.295 112.05) (end 151.115 109.23) (width 0.25) (layer "B.Cu") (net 18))
 (segment (start 177.8 121.92) (end 175.26 124.46) (width 0.25) (layer "B.Cu") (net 18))
 (segment (start 140.41 112.05) (end 148.295 112.05) (width 0.25) (layer "B.Cu") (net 18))
 (segment (start 187.96 116.84) (end 187.96 114.3) (width 0.25) (layer "B.Cu") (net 18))
 (segment (start 140.41 116.55) (end 133.91 116.55) (width 0.25) (layer "B.Cu") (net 18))
 (segment (start 180.37 101.69) (end 185.41 101.69) (width 0.25) (layer "B.Cu") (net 16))
 (segment (start 177.91 104.15) (end 180.37 101.69) (width 0.25) (layer "B.Cu") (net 16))
 (segment (start 185.41 101.69) (end 185.42 101.68) (width 0.25) (layer "B.Cu") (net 16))
 (segment (start 158.735 104.15) (end 177.91 104.15) (width 0.25) (layer "B.Cu") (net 16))
 (segment (start 180.27 106.69) (end 180.37 106.59) (width 0.25) (layer "B.Cu") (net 17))
 (segment (start 185.42 116.84) (end 180.37 111.79) (width 0.25) (layer "B.Cu") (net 17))
 (segment (start 158.735 106.69) (end 180.27 106.69) (width 0.25) (layer "B.Cu") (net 17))
 (segment (start 180.37 111.79) (end 180.37 106.59) (width 0.25) (layer "B.Cu") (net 17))
 (segment (start 157.21048 110.75452) (end 158.735 109.23) (width 0.25) (layer "F.Cu") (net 6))
 (segment (start 157.21048 117.10952) (end 157.21048 110.75452) (width 0.25) (layer "F.Cu") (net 6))
 (segment (start 137.16 137.16) (end 157.21048 117.10952) (width 0.25) (layer "F.Cu") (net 6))
 (segment (start 170.18 114.3) (end 165.11 109.23) (width 0.25) (layer "B.Cu") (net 6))
 (segment (start 170.18 114.3) (end 175.26 119.38) (width 0.25) (layer "B.Cu") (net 6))
 (segment (start 165.11 109.23) (end 158.735 109.23) (width 0.25) (layer "B.Cu") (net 6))
 (segment (start 142.24 116.84) (end 144.78 114.3) (width 0.25) (layer "B.Cu") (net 8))
 (segment (start 147.94 134.62) (end 147.94 132.7) (width 0.25) (layer "B.Cu") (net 8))
 (segment (start 148.585 114.3) (end 151.115 111.77) (width 0.25) (layer "B.Cu") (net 8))
 (segment (start 142.24 127) (end 142.24 116.84) (width 0.25) (layer "B.Cu") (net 8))
 (segment (start 147.94 132.7) (end 142.24 127) (width 0.25) (layer "B.Cu") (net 8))
 (segment (start 144.78 114.3) (end 148.585 114.3) (width 0.25) (layer "B.Cu") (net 8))
 (segment (start 144.78 116.84) (end 148.585 116.84) (width 0.25) (layer "B.Cu") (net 9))
 (segment (start 144.78 127) (end 144.78 116.84) (width 0.25) (layer "B.Cu") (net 9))
 (segment (start 148.585 116.84) (end 151.115 114.31) (width 0.25) (layer "B.Cu") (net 9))
 (segment (start 149.94 132.16) (end 144.78 127) (width 0.25) (layer "B.Cu") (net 9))
 (segment (start 149.94 134.62) (end 149.94 132.16) (width 0.25) (layer "B.Cu") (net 9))
 (segment (start 147.32 119.38) (end 149.85 116.85) (width 0.25) (layer "B.Cu") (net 10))
 (segment (start 151.94 131.62) (end 147.32 127) (width 0.25) (layer "B.Cu") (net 10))
 (segment (start 151.94 134.62) (end 151.94 131.62) (width 0.25) (layer "B.Cu") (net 10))
 (segment (start 147.32 127) (end 147.32 119.38) (width 0.25) (layer "B.Cu") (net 10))
 (segment (start 149.85 116.85) (end 151.115 116.85) (width 0.25) (layer "B.Cu") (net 10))
 (segment (start 153.94 131.08) (end 149.86 127) (width 0.25) (layer "B.Cu") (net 11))
 (segment (start 149.86 127) (end 149.86 121.92) (width 0.25) (layer "B.Cu") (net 11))
 (segment (start 149.86 121.92) (end 151.115 120.665) (width 0.25) (layer "B.Cu") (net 11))
 (segment (start 151.115 120.665) (end 151.115 119.39) (width 0.25) (layer "B.Cu") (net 11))
 (segment (start 153.94 134.62) (end 153.94 131.08) (width 0.25) (layer "B.Cu") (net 11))
 (segment (start 155.94 134.62) (end 155.94 122.185) (width 0.25) (layer "F.Cu") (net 12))
 (segment (start 155.94 122.185) (end 158.735 119.39) (width 0.25) (layer "F.Cu") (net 12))
 (segment (start 160.25952 118.37452) (end 158.735 116.85) (width 0.25) (layer "F.Cu") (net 13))
 (segment (start 157.94 134.62) (end 160.25952 132.30048) (width 0.25) (layer "F.Cu") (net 13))
 (segment (start 160.25952 132.30048) (end 160.25952 118.37452) (width 0.25) (layer "F.Cu") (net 13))
 (segment (start 162.56 132.08) (end 162.56 118.135) (width 0.25) (layer "F.Cu") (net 14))
 (segment (start 160.02 134.62) (end 162.56 132.08) (width 0.25) (layer "F.Cu") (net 14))
 (segment (start 159.94 134.62) (end 160.02 134.62) (width 0.25) (layer "F.Cu") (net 14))
 (segment (start 162.56 118.135) (end 158.735 114.31) (width 0.25) (layer "F.Cu") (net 14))
 (segment (start 161.94 134.62) (end 165.1 131.46) (width 0.25) (layer "F.Cu") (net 15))
 (segment (start 165.1 131.46) (end 165.1 118.135) (width 0.25) (layer "F.Cu") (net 15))
 (segment (start 165.1 118.135) (end 158.735 111.77) (width 0.25) (layer "F.Cu") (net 15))
 (segment (start 139.73452 105.56548) (end 154.77952 105.56548) (width 0.25) (layer "B.Cu") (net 1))
 (segment (start 154.77952 105.56548) (end 158.735 101.61) (width 0.25) (layer "B.Cu") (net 1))
 (segment (start 139.7 105.6) (end 139.73452 105.56548) (width 0.25) (layer "B.Cu") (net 1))
 (segment (start 153.645 93.98) (end 158.735 99.07) (width 0.25) (layer "B.Cu") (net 2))
 (segment (start 139.7 93.98) (end 153.645 93.98) (width 0.25) (layer "B.Cu") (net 2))
 (segment (start 139.7 103.6) (end 137.16 101.06) (width 0.25) (layer "B.Cu") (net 2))
 (segment (start 137.16 96.52) (end 139.7 93.98) (width 0.25) (layer "B.Cu") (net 2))
 (segment (start 137.16 101.06) (end 137.16 96.52) (width 0.25) (layer "B.Cu") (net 2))
 (segment (start 152.63952 102.075791) (end 152.63952 100.59452) (width 0.25) (layer "B.Cu") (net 3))
 (segment (start 139.7 101.6) (end 140.83452 102.73452) (width 0.25) (layer "B.Cu") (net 3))
 (segment (start 152.63952 100.59452) (end 151.115 99.07) (width 0.25) (layer "B.Cu") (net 3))
 (segment (start 140.83452 102.73452) (end 151.980791 102.73452) (width 0.25) (layer "B.Cu") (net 3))
 (segment (start 151.980791 102.73452) (end 152.63952 102.075791) (width 0.25) (layer "B.Cu") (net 3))
 (segment (start 149.105 99.6) (end 151.115 101.61) (width 0.25) (layer "B.Cu") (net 4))
 (segment (start 139.7 99.6) (end 149.105 99.6) (width 0.25) (layer "B.Cu") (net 4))
 (segment (start 139.7 97.6) (end 140.78 97.6) (width 0.25) (layer "F.Cu") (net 5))
 (segment (start 140.78 97.6) (end 147.32 104.14) (width 0.25) (layer "F.Cu") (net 5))
 (via (at 147.32 104.14) (size 0.8) (drill 0.4) (layers "F.Cu" "B.Cu") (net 5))
 (segment (start 147.32 104.14) (end 149.59048 104.14) (width 0.25) (layer "B.Cu") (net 5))
 (segment (start 163.69452 112.89452) (end 157.31952 112.89452) (width 0.25) (layer "B.Cu") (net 7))
 (segment (start 157.31952 112.89452) (end 151.115 106.69) (width 0.25) (layer "B.Cu") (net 7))
 (segment (start 170.18 119.38) (end 163.69452 112.89452) (width 0.25) (layer "B.Cu") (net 7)))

